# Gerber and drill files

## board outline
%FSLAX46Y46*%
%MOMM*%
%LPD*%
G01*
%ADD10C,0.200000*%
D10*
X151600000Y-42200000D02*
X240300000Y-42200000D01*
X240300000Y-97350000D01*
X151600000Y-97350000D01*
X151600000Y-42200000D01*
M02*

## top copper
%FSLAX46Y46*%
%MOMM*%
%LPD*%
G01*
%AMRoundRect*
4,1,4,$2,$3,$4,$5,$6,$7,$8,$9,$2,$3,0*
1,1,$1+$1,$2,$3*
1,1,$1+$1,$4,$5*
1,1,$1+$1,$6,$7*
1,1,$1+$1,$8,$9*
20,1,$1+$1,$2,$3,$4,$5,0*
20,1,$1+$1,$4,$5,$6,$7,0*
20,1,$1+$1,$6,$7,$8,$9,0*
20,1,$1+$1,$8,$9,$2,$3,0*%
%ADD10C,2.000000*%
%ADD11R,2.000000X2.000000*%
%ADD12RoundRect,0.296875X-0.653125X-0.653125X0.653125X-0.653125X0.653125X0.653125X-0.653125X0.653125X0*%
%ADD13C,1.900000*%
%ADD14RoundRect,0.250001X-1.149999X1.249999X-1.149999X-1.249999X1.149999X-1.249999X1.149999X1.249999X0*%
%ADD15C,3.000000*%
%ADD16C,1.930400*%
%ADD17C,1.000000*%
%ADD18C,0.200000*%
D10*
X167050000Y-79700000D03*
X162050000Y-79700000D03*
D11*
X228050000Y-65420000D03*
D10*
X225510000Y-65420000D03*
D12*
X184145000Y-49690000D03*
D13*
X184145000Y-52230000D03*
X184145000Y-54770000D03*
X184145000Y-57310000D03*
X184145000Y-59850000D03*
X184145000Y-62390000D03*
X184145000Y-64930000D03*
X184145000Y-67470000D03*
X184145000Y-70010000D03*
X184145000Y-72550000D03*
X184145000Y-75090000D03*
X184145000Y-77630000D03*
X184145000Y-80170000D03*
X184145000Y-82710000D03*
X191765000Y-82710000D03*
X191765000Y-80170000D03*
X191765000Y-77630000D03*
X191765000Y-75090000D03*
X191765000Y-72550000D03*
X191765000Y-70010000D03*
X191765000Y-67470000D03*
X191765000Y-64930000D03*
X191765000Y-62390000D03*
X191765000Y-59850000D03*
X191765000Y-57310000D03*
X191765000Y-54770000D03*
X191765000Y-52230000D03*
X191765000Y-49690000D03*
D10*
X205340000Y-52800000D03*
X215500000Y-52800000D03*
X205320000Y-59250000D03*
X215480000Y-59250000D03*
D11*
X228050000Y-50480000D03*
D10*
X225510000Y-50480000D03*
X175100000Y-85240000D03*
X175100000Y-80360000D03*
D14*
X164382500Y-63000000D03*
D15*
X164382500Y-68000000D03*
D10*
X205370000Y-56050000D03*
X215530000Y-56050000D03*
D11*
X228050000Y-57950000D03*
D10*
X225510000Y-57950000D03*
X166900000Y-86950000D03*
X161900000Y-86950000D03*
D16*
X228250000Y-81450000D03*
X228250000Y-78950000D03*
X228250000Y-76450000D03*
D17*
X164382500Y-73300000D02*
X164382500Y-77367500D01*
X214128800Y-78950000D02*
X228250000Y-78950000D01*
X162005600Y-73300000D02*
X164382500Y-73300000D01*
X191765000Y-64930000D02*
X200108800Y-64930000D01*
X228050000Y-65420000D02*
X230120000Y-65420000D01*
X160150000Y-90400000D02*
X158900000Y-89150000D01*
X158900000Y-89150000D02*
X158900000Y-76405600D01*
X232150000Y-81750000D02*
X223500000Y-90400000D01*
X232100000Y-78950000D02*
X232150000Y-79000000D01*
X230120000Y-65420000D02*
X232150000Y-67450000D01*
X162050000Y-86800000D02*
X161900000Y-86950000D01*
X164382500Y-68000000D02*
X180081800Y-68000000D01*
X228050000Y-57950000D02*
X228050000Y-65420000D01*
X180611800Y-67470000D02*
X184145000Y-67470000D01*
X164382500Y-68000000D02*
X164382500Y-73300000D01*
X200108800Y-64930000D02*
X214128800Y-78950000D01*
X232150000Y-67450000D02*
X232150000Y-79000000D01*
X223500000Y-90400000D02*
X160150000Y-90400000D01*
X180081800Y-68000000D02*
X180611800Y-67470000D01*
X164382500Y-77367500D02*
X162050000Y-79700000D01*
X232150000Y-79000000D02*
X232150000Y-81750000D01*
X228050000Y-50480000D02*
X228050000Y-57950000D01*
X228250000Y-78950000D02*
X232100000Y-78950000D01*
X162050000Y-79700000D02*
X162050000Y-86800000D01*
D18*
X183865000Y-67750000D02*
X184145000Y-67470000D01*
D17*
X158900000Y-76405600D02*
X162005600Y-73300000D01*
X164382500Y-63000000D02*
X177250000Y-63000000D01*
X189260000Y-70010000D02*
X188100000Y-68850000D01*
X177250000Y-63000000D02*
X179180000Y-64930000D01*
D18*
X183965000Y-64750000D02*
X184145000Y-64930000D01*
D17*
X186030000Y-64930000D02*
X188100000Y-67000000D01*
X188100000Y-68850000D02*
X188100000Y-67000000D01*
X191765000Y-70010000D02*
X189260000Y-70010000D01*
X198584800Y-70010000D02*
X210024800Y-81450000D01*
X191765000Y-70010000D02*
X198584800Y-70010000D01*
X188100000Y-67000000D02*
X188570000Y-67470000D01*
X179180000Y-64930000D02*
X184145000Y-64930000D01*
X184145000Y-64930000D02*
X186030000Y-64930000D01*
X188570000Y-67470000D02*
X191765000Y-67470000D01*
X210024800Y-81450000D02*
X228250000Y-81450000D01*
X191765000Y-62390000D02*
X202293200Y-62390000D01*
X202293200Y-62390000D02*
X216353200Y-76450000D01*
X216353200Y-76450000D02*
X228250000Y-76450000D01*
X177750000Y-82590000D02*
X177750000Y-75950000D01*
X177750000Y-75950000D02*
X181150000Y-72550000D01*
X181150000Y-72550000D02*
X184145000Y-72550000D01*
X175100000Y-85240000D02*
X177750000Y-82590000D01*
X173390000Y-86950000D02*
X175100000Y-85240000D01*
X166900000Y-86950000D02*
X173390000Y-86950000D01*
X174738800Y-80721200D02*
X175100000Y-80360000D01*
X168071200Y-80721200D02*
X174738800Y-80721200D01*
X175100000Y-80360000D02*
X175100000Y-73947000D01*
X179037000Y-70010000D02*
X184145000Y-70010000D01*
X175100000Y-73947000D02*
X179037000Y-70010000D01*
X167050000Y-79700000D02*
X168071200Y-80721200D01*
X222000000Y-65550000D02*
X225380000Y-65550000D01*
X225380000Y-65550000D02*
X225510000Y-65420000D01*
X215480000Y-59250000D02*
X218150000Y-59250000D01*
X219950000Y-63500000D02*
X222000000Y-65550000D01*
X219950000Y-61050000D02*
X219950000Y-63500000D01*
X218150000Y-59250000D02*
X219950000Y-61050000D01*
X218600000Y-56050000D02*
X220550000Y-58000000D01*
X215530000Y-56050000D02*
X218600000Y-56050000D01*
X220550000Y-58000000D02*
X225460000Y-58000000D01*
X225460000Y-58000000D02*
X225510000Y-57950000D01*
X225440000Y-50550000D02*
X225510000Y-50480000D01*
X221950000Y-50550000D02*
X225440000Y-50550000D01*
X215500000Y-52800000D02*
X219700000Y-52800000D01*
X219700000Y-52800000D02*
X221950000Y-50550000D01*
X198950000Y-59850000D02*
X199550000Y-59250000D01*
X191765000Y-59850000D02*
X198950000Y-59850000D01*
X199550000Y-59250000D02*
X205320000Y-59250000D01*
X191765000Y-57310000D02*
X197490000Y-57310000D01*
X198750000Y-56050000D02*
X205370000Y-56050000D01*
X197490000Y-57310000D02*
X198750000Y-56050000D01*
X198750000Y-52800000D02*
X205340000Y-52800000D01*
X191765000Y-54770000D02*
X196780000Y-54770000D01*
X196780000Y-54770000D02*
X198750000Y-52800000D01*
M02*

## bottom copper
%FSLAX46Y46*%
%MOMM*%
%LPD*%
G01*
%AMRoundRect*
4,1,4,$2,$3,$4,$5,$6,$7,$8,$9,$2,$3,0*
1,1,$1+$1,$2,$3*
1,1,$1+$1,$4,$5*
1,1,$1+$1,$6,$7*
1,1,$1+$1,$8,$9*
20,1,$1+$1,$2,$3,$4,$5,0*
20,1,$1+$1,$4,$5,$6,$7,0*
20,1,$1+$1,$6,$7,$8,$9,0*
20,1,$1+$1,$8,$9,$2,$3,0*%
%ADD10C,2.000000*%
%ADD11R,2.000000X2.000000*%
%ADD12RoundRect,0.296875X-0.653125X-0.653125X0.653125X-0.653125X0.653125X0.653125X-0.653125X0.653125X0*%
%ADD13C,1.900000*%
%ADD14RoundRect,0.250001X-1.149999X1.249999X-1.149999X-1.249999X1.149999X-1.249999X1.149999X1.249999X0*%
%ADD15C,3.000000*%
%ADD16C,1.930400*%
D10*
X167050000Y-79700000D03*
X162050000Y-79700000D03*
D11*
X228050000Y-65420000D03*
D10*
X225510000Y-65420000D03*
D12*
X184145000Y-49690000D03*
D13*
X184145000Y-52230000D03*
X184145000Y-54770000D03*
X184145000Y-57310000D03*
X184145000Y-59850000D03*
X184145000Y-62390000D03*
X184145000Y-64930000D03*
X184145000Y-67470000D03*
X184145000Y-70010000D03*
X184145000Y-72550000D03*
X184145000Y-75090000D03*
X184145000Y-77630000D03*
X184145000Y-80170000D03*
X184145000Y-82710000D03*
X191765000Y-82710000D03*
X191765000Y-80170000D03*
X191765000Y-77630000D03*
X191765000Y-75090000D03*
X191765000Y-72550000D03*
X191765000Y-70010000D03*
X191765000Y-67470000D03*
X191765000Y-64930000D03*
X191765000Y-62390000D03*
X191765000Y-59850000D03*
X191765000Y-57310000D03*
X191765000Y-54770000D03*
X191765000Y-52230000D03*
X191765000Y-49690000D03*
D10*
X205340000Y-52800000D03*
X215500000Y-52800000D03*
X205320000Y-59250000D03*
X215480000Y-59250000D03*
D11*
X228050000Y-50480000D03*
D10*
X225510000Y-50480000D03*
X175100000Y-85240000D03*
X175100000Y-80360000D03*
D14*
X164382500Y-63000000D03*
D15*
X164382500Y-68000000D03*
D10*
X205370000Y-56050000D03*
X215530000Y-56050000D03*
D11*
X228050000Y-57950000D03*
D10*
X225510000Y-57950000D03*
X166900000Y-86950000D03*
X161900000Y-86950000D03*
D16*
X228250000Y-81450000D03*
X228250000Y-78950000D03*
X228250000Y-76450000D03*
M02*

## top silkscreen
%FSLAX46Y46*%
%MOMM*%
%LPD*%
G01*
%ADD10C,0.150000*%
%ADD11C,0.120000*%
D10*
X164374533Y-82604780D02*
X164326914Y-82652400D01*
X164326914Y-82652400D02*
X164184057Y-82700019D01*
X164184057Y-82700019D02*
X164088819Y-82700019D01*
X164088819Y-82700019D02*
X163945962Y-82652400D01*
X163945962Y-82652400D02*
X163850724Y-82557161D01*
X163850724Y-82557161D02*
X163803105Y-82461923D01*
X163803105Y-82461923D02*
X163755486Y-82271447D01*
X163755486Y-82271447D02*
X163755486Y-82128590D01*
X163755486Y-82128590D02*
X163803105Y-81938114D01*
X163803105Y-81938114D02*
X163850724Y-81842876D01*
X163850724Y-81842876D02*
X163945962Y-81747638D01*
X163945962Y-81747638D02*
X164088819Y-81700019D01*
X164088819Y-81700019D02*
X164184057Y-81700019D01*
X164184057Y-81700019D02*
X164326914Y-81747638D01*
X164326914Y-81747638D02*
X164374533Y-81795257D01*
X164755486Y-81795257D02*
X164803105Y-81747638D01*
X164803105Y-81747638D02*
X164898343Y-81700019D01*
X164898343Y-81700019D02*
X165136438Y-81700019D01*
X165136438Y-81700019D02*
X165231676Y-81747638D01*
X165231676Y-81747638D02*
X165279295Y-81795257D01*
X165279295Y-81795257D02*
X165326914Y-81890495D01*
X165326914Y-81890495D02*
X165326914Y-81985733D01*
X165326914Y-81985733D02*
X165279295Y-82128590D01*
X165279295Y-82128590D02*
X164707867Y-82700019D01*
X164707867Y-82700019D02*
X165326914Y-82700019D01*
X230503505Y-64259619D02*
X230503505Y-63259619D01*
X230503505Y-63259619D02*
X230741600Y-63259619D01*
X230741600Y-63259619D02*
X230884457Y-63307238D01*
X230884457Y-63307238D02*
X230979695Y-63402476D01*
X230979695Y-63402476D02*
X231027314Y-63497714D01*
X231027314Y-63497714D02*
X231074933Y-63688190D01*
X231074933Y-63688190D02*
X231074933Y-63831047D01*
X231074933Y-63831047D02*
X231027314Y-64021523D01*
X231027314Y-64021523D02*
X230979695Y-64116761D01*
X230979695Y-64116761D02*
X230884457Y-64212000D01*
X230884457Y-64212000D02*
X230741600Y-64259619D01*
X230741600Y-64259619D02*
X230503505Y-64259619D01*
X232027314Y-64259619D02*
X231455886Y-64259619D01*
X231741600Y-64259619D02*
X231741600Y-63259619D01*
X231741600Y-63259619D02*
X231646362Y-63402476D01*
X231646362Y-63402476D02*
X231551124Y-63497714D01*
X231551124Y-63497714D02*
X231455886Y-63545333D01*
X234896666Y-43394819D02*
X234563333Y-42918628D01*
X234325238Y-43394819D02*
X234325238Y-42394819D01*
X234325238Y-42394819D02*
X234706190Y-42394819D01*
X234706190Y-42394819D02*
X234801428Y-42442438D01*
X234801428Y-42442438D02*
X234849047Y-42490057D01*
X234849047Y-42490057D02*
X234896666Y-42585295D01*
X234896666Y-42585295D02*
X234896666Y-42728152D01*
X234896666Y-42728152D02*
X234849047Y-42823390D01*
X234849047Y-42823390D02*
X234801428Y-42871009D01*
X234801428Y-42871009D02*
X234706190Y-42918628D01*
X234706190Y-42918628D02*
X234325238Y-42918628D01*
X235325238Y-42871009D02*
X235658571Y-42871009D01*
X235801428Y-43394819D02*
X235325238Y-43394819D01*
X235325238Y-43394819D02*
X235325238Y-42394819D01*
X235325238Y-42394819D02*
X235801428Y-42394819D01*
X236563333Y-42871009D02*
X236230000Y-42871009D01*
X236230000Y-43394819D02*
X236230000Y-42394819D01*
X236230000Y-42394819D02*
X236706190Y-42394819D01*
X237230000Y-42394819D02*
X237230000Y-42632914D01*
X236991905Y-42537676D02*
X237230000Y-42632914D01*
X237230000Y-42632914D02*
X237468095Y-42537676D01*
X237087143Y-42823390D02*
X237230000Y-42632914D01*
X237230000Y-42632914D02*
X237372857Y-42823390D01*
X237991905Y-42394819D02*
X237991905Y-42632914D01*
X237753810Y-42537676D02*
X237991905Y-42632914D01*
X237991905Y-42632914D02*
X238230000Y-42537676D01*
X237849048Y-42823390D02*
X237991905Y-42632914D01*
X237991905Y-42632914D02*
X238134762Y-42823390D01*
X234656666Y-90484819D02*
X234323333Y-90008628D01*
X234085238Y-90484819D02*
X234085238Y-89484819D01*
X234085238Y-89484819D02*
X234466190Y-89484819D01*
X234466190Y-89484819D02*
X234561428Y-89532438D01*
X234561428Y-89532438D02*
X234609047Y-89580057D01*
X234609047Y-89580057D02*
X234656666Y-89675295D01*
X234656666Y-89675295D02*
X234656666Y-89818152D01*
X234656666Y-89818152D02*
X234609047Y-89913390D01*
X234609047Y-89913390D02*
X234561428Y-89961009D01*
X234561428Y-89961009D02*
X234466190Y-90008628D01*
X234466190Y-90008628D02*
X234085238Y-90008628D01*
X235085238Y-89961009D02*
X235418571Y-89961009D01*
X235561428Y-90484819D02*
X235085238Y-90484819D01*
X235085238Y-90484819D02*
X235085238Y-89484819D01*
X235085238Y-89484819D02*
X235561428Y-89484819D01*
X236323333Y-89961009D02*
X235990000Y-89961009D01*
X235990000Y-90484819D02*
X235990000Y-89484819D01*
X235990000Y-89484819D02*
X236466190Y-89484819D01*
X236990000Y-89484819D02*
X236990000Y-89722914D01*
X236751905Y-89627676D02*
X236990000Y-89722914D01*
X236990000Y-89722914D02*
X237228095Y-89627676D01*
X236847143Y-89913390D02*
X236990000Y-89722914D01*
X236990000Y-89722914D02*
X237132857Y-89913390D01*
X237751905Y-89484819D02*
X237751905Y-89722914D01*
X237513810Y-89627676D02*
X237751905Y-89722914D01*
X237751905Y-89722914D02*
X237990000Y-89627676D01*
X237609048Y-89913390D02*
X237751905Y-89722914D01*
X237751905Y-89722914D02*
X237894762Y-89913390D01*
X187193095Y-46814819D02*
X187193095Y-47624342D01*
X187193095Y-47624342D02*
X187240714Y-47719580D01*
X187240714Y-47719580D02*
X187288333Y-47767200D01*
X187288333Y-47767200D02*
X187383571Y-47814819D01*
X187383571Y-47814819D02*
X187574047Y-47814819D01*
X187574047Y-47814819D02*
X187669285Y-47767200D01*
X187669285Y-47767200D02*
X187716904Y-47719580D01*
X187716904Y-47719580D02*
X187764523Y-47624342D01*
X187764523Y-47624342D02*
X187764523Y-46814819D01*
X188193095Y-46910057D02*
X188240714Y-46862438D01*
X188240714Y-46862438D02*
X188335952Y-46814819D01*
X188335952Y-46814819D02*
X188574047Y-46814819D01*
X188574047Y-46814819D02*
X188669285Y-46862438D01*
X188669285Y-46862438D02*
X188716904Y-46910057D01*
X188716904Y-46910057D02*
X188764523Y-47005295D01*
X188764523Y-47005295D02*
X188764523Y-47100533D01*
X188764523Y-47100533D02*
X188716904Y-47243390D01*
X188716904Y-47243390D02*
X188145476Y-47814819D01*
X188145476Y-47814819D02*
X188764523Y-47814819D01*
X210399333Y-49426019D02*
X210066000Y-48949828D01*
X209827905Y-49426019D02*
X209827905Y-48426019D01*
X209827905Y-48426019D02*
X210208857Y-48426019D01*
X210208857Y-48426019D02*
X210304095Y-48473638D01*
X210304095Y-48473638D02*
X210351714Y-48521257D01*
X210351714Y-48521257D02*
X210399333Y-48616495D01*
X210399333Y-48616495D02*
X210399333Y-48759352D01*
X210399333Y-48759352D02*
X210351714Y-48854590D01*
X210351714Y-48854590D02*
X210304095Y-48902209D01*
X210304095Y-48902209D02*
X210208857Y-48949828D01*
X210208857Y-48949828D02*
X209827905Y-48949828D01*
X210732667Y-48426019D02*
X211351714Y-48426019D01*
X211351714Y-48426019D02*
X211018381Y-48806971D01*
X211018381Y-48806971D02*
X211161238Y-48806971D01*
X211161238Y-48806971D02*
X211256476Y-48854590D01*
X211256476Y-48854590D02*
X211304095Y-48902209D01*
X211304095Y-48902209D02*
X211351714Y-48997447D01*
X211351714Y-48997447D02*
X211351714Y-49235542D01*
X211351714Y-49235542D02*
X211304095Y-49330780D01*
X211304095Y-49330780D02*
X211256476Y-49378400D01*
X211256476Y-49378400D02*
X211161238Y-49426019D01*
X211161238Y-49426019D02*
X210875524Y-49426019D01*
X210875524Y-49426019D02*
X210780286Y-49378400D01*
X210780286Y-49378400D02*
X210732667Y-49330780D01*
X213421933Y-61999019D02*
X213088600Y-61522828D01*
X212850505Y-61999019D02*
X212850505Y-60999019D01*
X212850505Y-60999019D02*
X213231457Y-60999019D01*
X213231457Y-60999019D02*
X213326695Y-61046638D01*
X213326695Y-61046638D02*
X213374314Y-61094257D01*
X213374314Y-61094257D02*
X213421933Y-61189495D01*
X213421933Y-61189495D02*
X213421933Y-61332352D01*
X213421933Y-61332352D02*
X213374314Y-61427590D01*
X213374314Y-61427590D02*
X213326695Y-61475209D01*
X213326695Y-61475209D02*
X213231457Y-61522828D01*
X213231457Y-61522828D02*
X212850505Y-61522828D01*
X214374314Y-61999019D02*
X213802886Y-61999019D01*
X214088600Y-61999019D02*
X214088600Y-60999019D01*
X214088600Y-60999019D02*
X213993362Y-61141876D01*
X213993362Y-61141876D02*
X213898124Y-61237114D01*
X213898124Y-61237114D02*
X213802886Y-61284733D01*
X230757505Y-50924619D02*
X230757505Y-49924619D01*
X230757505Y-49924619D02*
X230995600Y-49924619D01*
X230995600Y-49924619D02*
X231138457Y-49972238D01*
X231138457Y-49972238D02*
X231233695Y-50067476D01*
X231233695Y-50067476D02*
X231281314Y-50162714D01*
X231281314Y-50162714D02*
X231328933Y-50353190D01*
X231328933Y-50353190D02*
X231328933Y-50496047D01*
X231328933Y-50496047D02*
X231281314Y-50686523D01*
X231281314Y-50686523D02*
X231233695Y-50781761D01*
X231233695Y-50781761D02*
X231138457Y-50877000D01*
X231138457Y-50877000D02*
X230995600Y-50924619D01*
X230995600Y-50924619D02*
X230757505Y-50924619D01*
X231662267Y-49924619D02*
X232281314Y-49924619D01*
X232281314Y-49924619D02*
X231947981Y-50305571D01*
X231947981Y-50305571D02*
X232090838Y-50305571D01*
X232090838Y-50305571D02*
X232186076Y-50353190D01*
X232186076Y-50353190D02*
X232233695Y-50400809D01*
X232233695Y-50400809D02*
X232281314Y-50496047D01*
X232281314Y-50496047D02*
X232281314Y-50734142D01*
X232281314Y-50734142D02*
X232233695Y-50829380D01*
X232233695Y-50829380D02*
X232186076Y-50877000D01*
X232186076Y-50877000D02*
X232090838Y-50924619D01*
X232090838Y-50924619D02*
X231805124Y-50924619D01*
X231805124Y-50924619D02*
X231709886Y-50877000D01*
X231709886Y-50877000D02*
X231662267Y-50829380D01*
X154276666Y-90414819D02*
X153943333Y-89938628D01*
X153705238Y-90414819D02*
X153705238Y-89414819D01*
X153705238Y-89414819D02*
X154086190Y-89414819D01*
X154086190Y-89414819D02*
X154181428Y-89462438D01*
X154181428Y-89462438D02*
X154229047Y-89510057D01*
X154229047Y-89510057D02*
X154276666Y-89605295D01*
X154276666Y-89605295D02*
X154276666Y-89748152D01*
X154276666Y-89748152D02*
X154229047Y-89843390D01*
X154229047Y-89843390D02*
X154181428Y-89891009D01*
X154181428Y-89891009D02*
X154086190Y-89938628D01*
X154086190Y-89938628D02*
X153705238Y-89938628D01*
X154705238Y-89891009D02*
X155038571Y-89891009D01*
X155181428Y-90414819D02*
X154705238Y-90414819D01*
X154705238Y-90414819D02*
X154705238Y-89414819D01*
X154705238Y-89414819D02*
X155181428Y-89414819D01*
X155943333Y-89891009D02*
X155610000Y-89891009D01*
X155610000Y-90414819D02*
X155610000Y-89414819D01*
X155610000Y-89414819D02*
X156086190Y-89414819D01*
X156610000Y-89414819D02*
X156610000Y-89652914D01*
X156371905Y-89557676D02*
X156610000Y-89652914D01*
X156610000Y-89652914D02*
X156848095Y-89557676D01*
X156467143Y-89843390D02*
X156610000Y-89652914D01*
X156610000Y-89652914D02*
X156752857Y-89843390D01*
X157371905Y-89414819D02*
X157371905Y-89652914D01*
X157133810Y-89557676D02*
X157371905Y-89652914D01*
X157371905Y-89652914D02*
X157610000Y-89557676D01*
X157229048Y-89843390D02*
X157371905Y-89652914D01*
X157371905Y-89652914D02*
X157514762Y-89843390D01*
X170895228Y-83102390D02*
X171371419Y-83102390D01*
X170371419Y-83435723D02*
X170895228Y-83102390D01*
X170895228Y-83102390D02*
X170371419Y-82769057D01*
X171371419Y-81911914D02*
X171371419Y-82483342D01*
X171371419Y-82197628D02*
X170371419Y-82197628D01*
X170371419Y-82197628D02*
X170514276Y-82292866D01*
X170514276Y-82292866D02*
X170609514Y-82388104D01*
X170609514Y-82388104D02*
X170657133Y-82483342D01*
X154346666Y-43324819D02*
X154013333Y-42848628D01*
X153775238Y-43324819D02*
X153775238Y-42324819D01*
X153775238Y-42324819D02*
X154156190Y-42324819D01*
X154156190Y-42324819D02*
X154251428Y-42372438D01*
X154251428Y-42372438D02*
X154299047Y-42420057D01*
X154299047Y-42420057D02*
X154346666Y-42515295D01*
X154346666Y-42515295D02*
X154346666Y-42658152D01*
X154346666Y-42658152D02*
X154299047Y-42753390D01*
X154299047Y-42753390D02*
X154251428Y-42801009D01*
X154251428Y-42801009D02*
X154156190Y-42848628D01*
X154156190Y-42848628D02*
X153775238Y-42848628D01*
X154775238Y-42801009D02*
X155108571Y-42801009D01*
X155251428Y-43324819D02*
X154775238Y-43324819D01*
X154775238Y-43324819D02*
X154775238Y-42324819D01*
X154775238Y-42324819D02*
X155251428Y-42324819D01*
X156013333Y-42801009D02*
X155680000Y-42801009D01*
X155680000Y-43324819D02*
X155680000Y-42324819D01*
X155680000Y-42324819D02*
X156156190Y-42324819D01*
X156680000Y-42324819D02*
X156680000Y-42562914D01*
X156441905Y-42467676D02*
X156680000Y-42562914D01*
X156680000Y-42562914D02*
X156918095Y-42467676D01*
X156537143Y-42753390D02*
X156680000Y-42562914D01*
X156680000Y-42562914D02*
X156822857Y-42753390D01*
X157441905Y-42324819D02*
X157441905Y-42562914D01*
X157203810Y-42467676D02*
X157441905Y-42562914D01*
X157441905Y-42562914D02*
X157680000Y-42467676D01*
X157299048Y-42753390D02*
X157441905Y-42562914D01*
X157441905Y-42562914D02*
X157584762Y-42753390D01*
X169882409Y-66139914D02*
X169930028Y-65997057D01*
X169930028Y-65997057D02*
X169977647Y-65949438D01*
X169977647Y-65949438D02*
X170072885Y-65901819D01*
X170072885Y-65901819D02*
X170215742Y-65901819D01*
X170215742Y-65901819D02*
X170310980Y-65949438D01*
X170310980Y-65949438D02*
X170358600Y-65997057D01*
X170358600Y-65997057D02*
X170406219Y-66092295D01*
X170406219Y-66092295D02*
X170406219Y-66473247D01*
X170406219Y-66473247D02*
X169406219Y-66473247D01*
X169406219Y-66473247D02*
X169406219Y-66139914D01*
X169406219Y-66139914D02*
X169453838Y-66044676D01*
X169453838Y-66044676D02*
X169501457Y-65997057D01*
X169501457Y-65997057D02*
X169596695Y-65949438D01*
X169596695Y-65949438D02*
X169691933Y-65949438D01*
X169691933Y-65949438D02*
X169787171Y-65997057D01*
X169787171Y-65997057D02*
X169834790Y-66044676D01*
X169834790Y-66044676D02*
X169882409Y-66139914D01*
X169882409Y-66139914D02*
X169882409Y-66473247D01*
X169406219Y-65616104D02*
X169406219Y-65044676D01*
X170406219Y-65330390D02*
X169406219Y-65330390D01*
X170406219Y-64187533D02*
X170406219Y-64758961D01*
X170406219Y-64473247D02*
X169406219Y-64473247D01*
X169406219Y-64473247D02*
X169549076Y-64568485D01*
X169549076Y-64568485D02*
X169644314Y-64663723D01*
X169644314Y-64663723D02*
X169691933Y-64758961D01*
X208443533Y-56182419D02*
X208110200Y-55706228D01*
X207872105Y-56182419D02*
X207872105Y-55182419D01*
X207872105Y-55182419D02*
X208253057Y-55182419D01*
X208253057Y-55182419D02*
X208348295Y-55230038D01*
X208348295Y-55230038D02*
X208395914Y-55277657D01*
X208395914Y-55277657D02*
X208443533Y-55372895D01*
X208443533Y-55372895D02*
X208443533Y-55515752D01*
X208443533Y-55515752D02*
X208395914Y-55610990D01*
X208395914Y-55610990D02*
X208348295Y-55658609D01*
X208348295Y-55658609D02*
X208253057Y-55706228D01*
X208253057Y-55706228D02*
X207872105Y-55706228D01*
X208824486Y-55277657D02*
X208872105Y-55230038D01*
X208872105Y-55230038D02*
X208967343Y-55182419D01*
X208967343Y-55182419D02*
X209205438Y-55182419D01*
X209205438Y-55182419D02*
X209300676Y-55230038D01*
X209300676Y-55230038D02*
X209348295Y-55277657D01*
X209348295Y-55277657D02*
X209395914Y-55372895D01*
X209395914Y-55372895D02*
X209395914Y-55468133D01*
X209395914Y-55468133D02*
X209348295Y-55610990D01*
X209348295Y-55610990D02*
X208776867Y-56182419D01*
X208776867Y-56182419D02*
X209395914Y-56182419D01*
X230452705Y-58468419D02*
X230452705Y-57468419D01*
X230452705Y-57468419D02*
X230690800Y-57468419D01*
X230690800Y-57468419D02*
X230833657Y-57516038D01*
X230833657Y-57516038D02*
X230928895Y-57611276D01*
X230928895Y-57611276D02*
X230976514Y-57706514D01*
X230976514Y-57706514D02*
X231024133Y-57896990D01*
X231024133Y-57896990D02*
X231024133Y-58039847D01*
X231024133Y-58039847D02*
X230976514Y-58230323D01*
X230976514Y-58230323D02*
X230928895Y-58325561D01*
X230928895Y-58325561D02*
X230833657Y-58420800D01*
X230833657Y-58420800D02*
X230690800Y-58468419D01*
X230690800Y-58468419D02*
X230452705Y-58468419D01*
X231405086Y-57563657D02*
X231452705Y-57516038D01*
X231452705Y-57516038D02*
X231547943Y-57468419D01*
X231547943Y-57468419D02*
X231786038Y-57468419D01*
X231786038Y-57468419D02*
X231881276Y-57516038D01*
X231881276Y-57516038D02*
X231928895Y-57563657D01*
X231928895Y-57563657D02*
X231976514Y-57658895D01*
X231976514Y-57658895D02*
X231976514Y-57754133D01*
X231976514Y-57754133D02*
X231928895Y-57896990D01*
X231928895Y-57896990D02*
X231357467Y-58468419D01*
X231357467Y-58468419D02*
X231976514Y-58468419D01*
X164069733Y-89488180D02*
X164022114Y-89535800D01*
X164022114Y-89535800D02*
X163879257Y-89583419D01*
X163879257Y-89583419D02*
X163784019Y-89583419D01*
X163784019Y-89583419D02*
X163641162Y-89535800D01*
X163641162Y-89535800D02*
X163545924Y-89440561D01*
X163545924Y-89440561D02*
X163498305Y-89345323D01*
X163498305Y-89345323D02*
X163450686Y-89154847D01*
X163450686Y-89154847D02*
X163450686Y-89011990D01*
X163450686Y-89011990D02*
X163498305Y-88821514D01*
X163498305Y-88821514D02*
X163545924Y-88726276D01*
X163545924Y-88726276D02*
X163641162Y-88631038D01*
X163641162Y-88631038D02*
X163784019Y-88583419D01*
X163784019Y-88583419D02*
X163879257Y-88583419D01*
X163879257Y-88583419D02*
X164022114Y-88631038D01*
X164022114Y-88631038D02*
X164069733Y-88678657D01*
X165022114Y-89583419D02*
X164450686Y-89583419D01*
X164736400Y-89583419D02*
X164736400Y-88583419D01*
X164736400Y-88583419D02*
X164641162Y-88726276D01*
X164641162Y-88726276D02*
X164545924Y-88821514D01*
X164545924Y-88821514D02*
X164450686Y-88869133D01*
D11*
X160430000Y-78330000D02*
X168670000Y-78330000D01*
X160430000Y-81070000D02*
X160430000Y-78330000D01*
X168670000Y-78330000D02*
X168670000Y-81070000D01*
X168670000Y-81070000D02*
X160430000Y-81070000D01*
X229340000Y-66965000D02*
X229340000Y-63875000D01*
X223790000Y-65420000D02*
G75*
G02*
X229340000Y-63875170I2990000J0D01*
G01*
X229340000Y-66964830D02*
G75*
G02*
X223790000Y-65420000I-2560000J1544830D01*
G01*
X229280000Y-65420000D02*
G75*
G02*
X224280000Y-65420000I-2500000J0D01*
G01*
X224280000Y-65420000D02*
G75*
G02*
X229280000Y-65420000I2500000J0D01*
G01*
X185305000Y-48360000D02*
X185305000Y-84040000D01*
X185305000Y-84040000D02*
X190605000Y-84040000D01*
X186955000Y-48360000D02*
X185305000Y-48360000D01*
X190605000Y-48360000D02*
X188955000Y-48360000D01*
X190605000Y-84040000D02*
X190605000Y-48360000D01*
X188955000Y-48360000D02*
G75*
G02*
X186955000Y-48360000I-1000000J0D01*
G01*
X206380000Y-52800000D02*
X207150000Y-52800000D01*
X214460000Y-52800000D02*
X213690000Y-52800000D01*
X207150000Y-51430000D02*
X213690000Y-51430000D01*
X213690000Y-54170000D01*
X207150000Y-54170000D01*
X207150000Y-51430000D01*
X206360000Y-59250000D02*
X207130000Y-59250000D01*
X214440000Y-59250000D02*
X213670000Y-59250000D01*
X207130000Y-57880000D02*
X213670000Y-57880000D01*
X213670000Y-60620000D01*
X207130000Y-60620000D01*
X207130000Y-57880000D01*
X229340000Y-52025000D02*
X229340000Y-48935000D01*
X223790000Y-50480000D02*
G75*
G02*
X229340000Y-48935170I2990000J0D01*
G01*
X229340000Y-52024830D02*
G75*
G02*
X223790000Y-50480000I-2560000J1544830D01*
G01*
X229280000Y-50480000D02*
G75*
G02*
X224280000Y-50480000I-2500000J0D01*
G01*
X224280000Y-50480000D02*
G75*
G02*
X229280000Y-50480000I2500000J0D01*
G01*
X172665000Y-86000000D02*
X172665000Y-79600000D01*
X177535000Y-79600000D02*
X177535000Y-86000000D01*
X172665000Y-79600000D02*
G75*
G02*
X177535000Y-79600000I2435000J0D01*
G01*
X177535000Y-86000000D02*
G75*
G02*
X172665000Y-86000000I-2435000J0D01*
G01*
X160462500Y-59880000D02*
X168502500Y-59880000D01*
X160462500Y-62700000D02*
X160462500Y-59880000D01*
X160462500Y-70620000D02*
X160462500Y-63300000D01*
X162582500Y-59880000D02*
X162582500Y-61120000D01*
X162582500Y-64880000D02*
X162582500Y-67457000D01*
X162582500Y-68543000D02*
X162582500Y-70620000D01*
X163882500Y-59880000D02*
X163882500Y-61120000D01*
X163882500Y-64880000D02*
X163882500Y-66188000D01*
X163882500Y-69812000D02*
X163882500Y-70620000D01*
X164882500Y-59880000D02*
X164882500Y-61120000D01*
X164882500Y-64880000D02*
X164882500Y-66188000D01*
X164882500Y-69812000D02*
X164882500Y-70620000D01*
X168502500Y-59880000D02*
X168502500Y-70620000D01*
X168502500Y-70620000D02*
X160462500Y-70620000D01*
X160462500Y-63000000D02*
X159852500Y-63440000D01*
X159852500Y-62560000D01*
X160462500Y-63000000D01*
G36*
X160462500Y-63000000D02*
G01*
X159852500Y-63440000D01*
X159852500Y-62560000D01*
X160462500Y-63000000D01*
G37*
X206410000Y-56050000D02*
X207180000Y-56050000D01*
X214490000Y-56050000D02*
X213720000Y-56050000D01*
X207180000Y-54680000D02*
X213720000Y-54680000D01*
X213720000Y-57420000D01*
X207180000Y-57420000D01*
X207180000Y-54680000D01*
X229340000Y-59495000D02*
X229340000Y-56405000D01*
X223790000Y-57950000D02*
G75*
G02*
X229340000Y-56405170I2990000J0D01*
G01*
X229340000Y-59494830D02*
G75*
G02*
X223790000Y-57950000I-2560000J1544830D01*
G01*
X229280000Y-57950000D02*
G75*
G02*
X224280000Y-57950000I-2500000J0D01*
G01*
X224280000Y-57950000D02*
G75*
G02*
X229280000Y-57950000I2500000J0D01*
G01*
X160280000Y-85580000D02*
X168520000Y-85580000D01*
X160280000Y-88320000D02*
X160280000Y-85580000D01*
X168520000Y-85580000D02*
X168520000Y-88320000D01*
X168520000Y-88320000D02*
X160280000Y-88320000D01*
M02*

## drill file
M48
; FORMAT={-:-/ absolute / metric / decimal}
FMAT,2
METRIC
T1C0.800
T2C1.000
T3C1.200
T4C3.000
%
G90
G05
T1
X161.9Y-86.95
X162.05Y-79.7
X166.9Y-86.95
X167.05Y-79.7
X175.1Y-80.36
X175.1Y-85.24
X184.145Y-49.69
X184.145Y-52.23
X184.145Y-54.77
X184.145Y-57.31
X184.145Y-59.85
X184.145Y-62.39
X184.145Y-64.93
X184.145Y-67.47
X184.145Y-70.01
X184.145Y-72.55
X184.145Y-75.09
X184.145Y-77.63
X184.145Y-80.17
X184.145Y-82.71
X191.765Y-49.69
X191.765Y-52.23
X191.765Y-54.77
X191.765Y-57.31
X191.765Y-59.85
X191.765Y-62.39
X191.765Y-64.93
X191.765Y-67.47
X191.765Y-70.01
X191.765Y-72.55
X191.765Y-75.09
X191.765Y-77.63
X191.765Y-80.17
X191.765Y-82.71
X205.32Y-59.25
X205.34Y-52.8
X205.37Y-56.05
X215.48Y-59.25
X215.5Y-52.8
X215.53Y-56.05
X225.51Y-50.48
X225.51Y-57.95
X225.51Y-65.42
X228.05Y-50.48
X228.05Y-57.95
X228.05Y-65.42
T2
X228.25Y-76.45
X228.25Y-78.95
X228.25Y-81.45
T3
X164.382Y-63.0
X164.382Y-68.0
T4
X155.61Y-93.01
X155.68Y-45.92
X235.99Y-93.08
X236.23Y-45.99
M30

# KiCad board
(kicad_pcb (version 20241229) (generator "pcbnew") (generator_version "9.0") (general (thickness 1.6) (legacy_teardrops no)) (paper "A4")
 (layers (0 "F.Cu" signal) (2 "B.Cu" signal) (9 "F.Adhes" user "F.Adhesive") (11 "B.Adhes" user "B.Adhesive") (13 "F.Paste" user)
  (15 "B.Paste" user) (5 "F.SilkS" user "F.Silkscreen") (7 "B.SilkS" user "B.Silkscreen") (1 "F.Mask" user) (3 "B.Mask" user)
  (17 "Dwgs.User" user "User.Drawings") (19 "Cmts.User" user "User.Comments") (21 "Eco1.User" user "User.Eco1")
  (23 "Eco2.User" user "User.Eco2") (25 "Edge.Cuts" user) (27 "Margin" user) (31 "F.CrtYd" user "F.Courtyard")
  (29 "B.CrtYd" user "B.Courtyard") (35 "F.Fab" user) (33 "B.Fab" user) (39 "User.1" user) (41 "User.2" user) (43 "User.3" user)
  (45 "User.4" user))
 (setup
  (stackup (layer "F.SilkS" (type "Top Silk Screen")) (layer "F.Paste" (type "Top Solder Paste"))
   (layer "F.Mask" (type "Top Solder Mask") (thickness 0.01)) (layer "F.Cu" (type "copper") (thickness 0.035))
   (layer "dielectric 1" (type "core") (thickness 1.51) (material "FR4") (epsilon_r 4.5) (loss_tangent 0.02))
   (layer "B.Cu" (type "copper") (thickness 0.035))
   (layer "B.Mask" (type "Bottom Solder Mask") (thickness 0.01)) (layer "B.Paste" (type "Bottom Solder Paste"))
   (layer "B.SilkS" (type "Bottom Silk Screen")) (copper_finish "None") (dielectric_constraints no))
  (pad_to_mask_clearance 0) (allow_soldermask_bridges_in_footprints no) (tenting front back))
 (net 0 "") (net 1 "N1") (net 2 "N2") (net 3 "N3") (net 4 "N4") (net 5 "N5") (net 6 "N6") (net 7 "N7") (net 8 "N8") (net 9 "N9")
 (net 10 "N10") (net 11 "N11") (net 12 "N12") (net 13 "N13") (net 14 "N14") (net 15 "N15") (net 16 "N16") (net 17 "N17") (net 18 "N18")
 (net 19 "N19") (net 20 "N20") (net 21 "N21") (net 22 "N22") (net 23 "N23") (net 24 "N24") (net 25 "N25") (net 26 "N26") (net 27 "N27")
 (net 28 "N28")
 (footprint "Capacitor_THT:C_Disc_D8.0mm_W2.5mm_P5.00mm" (layer "F.Cu") (at 167.05 79.7 180)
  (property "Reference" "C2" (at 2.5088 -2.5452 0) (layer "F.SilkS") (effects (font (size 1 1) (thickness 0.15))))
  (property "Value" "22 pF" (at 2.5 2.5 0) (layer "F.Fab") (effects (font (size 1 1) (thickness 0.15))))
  (fp_line (start 6.62 1.37) (end -1.62 1.37) (stroke (width 0.12) (type solid)) (layer "F.SilkS"))
  (fp_line (start 6.62 -1.37) (end 6.62 1.37) (stroke (width 0.12) (type solid)) (layer "F.SilkS"))
  (fp_line (start -1.62 1.37) (end -1.62 -1.37) (stroke (width 0.12) (type solid)) (layer "F.SilkS"))
  (fp_line (start -1.62 -1.37) (end 6.62 -1.37) (stroke (width 0.12) (type solid)) (layer "F.SilkS"))
  (pad "1" thru_hole circle (at 0 0 180) (size 2 2) (drill 0.8) (layers "*.Cu" "*.Mask") (remove_unused_layers no) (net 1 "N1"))
  (pad "2" thru_hole circle (at 5 0 180) (size 2 2) (drill 0.8) (layers "*.Cu" "*.Mask") (remove_unused_layers no) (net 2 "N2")))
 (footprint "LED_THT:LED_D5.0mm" (layer "F.Cu") (at 228.05 65.42 180)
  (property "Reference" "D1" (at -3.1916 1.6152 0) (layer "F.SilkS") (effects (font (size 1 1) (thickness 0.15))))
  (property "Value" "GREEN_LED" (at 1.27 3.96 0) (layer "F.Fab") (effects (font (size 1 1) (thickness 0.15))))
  (fp_line (start -1.29 -1.545) (end -1.29 1.545) (stroke (width 0.12) (type solid)) (layer "F.SilkS"))
  (fp_arc (start 4.26 0) (mid 2.071779 2.880495) (end -1.29 1.54483) (stroke (width 0.12) (type solid)) (layer "F.SilkS"))
  (fp_arc (start -1.29 -1.54483) (mid 2.071779 -2.880495) (end 4.26 0) (stroke (width 0.12) (type solid)) (layer "F.SilkS"))
  (fp_circle (center 1.27 0) (end 3.77 0) (stroke (width 0.12) (type solid)) (fill no) (layer "F.SilkS"))
  (pad "1" thru_hole rect (at 0 0 180) (size 2 2) (drill 0.8) (layers "*.Cu" "*.Mask") (remove_unused_layers no) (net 2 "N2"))
  (pad "2" thru_hole circle (at 2.54 0 180) (size 2 2) (drill 0.8) (layers "*.Cu" "*.Mask") (remove_unused_layers no) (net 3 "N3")))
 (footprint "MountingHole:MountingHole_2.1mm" (layer "F.Cu") (at 236.23 45.99)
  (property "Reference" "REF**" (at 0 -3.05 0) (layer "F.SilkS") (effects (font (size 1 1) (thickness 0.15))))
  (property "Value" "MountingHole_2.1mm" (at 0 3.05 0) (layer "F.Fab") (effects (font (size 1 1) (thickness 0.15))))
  (pad "" np_thru_hole circle (at 0 0) (size 2.1 2.1) (drill 3) (layers "*.Cu" "*.Mask")))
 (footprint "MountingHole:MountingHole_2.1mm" (layer "F.Cu") (at 235.99 93.08)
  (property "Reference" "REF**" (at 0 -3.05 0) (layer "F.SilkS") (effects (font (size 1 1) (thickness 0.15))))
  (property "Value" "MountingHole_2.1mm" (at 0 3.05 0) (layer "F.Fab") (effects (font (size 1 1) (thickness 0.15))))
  (pad "" np_thru_hole circle (at 0 0) (size 2.1 2.1) (drill 3) (layers "*.Cu" "*.Mask")))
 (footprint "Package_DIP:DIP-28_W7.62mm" (layer "F.Cu") (at 184.145 49.69)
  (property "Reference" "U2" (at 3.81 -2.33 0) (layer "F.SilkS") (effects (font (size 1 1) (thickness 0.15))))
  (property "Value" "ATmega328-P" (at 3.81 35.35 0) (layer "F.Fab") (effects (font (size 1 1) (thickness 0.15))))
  (fp_line (start 1.16 -1.33) (end 1.16 34.35) (stroke (width 0.12) (type solid)) (layer "F.SilkS"))
  (fp_line (start 1.16 34.35) (end 6.46 34.35) (stroke (width 0.12) (type solid)) (layer "F.SilkS"))
  (fp_line (start 2.81 -1.33) (end 1.16 -1.33) (stroke (width 0.12) (type solid)) (layer "F.SilkS"))
  (fp_line (start 6.46 -1.33) (end 4.81 -1.33) (stroke (width 0.12) (type solid)) (layer "F.SilkS"))
  (fp_line (start 6.46 34.35) (end 6.46 -1.33) (stroke (width 0.12) (type solid)) (layer "F.SilkS"))
  (fp_arc (start 4.81 -1.33) (mid 3.81 -0.33) (end 2.81 -1.33) (stroke (width 0.12) (type solid)) (layer "F.SilkS"))
  (pad "1" thru_hole roundrect (at 0 0) (size 1.9 1.9) (drill 0.8) (layers "*.Cu" "*.Mask") (remove_unused_layers no)
   (roundrect_rratio 0.15625) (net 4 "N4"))
  (pad "2" thru_hole circle (at 0 2.54) (size 1.9 1.9) (drill 0.8) (layers "*.Cu" "*.Mask") (remove_unused_layers no) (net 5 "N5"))
  (pad "3" thru_hole circle (at 0 5.08) (size 1.9 1.9) (drill 0.8) (layers "*.Cu" "*.Mask") (remove_unused_layers no) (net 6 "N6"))
  (pad "4" thru_hole circle (at 0 7.62) (size 1.9 1.9) (drill 0.8) (layers "*.Cu" "*.Mask") (remove_unused_layers no) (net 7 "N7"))
  (pad "5" thru_hole circle (at 0 10.16) (size 1.9 1.9) (drill 0.8) (layers "*.Cu" "*.Mask") (remove_unused_layers no) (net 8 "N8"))
  (pad "6" thru_hole circle (at 0 12.7) (size 1.9 1.9) (drill 0.8) (layers "*.Cu" "*.Mask") (remove_unused_layers no) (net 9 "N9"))
  (pad "7" thru_hole circle (at 0 15.24) (size 1.9 1.9) (drill 0.8) (layers "*.Cu" "*.Mask") (remove_unused_layers no) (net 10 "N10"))
  (pad "8" thru_hole circle (at 0 17.78) (size 1.9 1.9) (drill 0.8) (layers "*.Cu" "*.Mask") (remove_unused_layers no) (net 2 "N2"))
  (pad "9" thru_hole circle (at 0 20.32) (size 1.9 1.9) (drill 0.8) (layers "*.Cu" "*.Mask") (remove_unused_layers no) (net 1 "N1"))
  (pad "10" thru_hole circle (at 0 22.86) (size 1.9 1.9) (drill 0.8) (layers "*.Cu" "*.Mask") (remove_unused_layers no) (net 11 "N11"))
  (pad "11" thru_hole circle (at 0 25.4) (size 1.9 1.9) (drill 0.8) (layers "*.Cu" "*.Mask") (remove_unused_layers no) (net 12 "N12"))
  (pad "12" thru_hole circle (at 0 27.94) (size 1.9 1.9) (drill 0.8) (layers "*.Cu" "*.Mask") (remove_unused_layers no) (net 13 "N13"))
  (pad "13" thru_hole circle (at 0 30.48) (size 1.9 1.9) (drill 0.8) (layers "*.Cu" "*.Mask") (remove_unused_layers no) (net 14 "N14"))
  (pad "14" thru_hole circle (at 0 33.02) (size 1.9 1.9) (drill 0.8) (layers "*.Cu" "*.Mask") (remove_unused_layers no) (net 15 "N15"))
  (pad "15" thru_hole circle (at 7.62 33.02) (size 1.9 1.9) (drill 0.8) (layers "*.Cu" "*.Mask") (remove_unused_layers no) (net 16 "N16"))
  (pad "16" thru_hole circle (at 7.62 30.48) (size 1.9 1.9) (drill 0.8) (layers "*.Cu" "*.Mask") (remove_unused_layers no) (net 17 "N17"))
  (pad "17" thru_hole circle (at 7.62 27.94) (size 1.9 1.9) (drill 0.8) (layers "*.Cu" "*.Mask") (remove_unused_layers no) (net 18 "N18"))
  (pad "18" thru_hole circle (at 7.62 25.4) (size 1.9 1.9) (drill 0.8) (layers "*.Cu" "*.Mask") (remove_unused_layers no) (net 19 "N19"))
  (pad "19" thru_hole circle (at 7.62 22.86) (size 1.9 1.9) (drill 0.8) (layers "*.Cu" "*.Mask") (remove_unused_layers no) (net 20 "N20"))
  (pad "20" thru_hole circle (at 7.62 20.32) (size 1.9 1.9) (drill 0.8) (layers "*.Cu" "*.Mask") (remove_unused_layers no) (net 10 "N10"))
  (pad "21" thru_hole circle (at 7.62 17.78) (size 1.9 1.9) (drill 0.8) (layers "*.Cu" "*.Mask") (remove_unused_layers no) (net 10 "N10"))
  (pad "22" thru_hole circle (at 7.62 15.24) (size 1.9 1.9) (drill 0.8) (layers "*.Cu" "*.Mask") (remove_unused_layers no) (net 2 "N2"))
  (pad "23" thru_hole circle (at 7.62 12.7) (size 1.9 1.9) (drill 0.8) (layers "*.Cu" "*.Mask") (remove_unused_layers no) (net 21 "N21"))
  (pad "24" thru_hole circle (at 7.62 10.16) (size 1.9 1.9) (drill 0.8) (layers "*.Cu" "*.Mask") (remove_unused_layers no) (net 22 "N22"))
  (pad "25" thru_hole circle (at 7.62 7.62) (size 1.9 1.9) (drill 0.8) (layers "*.Cu" "*.Mask") (remove_unused_layers no) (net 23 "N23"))
  (pad "26" thru_hole circle (at 7.62 5.08) (size 1.9 1.9) (drill 0.8) (layers "*.Cu" "*.Mask") (remove_unused_layers no) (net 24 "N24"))
  (pad "27" thru_hole circle (at 7.62 2.54) (size 1.9 1.9) (drill 0.8) (layers "*.Cu" "*.Mask") (remove_unused_layers no) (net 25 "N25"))
  (pad "28" thru_hole circle (at 7.62 0) (size 1.9 1.9) (drill 0.8) (layers "*.Cu" "*.Mask") (remove_unused_layers no) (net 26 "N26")))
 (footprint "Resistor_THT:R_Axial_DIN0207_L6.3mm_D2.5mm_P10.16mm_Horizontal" (layer "F.Cu") (at 205.34 52.8)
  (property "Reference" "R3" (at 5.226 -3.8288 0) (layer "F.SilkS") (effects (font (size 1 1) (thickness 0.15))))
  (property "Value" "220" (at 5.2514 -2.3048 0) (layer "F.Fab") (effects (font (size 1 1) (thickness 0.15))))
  (fp_line (start 1.04 0) (end 1.81 0) (stroke (width 0.12) (type solid)) (layer "F.SilkS"))
  (fp_line (start 9.12 0) (end 8.35 0) (stroke (width 0.12) (type solid)) (layer "F.SilkS"))
  (fp_rect (start 1.81 -1.37) (end 8.35 1.37) (stroke (width 0.12) (type solid)) (fill no) (layer "F.SilkS"))
  (pad "1" thru_hole circle (at 0 0) (size 2 2) (drill 0.8) (layers "*.Cu" "*.Mask") (remove_unused_layers no) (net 24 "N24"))
  (pad "2" thru_hole circle (at 10.16 0) (size 2 2) (drill 0.8) (layers "*.Cu" "*.Mask") (remove_unused_layers no) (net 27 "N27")))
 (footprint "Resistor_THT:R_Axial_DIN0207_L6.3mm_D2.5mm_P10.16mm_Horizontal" (layer "F.Cu") (at 205.32 59.25)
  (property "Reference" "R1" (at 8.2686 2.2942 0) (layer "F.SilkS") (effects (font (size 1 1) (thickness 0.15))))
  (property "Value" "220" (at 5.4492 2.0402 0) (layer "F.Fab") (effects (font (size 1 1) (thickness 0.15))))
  (fp_line (start 1.04 0) (end 1.81 0) (stroke (width 0.12) (type solid)) (layer "F.SilkS"))
  (fp_line (start 9.12 0) (end 8.35 0) (stroke (width 0.12) (type solid)) (layer "F.SilkS"))
  (fp_rect (start 1.81 -1.37) (end 8.35 1.37) (stroke (width 0.12) (type solid)) (fill no) (layer "F.SilkS"))
  (pad "1" thru_hole circle (at 0 0) (size 2 2) (drill 0.8) (layers "*.Cu" "*.Mask") (remove_unused_layers no) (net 22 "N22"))
  (pad "2" thru_hole circle (at 10.16 0) (size 2 2) (drill 0.8) (layers "*.Cu" "*.Mask") (remove_unused_layers no) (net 3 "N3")))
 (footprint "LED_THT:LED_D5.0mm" (layer "F.Cu") (at 228.05 50.48 180)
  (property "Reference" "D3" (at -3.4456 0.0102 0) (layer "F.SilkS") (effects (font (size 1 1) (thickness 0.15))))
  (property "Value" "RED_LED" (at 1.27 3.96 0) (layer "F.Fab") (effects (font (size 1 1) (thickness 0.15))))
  (fp_line (start -1.29 -1.545) (end -1.29 1.545) (stroke (width 0.12) (type solid)) (layer "F.SilkS"))
  (fp_arc (start 4.26 0) (mid 2.071779 2.880495) (end -1.29 1.54483) (stroke (width 0.12) (type solid)) (layer "F.SilkS"))
  (fp_arc (start -1.29 -1.54483) (mid 2.071779 -2.880495) (end 4.26 0) (stroke (width 0.12) (type solid)) (layer "F.SilkS"))
  (fp_circle (center 1.27 0) (end 3.77 0) (stroke (width 0.12) (type solid)) (fill no) (layer "F.SilkS"))
  (pad "1" thru_hole rect (at 0 0 180) (size 2 2) (drill 0.8) (layers "*.Cu" "*.Mask") (remove_unused_layers no) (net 2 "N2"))
  (pad "2" thru_hole circle (at 2.54 0 180) (size 2 2) (drill 0.8) (layers "*.Cu" "*.Mask") (remove_unused_layers no) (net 27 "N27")))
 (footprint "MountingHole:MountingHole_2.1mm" (layer "F.Cu") (at 155.61 93.01)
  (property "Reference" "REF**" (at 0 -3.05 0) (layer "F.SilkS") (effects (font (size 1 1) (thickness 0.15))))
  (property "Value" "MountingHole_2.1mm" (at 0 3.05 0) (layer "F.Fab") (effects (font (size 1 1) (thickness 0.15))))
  (pad "" np_thru_hole circle (at 0 0) (size 2.1 2.1) (drill 3) (layers "*.Cu" "*.Mask")))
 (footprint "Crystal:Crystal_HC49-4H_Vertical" (layer "F.Cu") (at 175.1 85.24 90)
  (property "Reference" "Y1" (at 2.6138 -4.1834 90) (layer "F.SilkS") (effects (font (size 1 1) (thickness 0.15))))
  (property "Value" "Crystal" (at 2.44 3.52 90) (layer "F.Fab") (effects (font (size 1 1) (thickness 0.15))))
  (fp_line (start -0.76 -2.435) (end 5.64 -2.435) (stroke (width 0.12) (type solid)) (layer "F.SilkS"))
  (fp_line (start 5.64 2.435) (end -0.76 2.435) (stroke (width 0.12) (type solid)) (layer "F.SilkS"))
  (fp_arc (start 5.64 -2.435) (mid 8.075 0) (end 5.64 2.435) (stroke (width 0.12) (type solid)) (layer "F.SilkS"))
  (fp_arc (start -0.76 2.435) (mid -3.195 0) (end -0.76 -2.435) (stroke (width 0.12) (type solid)) (layer "F.SilkS"))
  (pad "1" thru_hole circle (at 0 0 90) (size 2 2) (drill 0.8) (layers "*.Cu" "*.Mask") (remove_unused_layers no) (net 11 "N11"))
  (pad "2" thru_hole circle (at 4.88 0 90) (size 2 2) (drill 0.8) (layers "*.Cu" "*.Mask") (remove_unused_layers no) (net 1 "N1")))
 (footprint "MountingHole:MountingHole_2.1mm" (layer "F.Cu") (at 155.68 45.92)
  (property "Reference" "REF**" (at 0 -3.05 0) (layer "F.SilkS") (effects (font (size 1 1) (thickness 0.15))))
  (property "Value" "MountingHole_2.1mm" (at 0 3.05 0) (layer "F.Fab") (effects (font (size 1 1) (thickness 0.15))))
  (pad "" np_thru_hole circle (at 0 0) (size 2.1 2.1) (drill 3) (layers "*.Cu" "*.Mask")))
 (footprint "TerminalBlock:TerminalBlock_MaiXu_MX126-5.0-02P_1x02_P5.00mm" (layer "F.Cu") (at 164.3825 63 -90)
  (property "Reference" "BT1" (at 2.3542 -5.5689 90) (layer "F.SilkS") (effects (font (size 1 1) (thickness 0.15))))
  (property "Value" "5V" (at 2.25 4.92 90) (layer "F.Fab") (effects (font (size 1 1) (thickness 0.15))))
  (fp_line (start -3.12 3.92) (end -3.12 -4.12) (stroke (width 0.12) (type solid)) (layer "F.SilkS"))
  (fp_line (start -0.3 3.92) (end -3.12 3.92) (stroke (width 0.12) (type solid)) (layer "F.SilkS"))
  (fp_line (start 7.62 3.92) (end 0.3 3.92) (stroke (width 0.12) (type solid)) (layer "F.SilkS"))
  (fp_line (start -3.12 1.8) (end -1.88 1.8) (stroke (width 0.12) (type solid)) (layer "F.SilkS"))
  (fp_line (start 1.88 1.8) (end 4.457 1.8) (stroke (width 0.12) (type solid)) (layer "F.SilkS"))
  (fp_line (start 5.543 1.8) (end 7.62 1.8) (stroke (width 0.12) (type solid)) (layer "F.SilkS"))
  (fp_line (start -3.12 0.5) (end -1.88 0.5) (stroke (width 0.12) (type solid)) (layer "F.SilkS"))
  (fp_line (start 1.88 0.5) (end 3.188 0.5) (stroke (width 0.12) (type solid)) (layer "F.SilkS"))
  (fp_line (start 6.812 0.5) (end 7.62 0.5) (stroke (width 0.12) (type solid)) (layer "F.SilkS"))
  (fp_line (start -3.12 -0.5) (end -1.88 -0.5) (stroke (width 0.12) (type solid)) (layer "F.SilkS"))
  (fp_line (start 1.88 -0.5) (end 3.188 -0.5) (stroke (width 0.12) (type solid)) (layer "F.SilkS"))
  (fp_line (start 6.812 -0.5) (end 7.62 -0.5) (stroke (width 0.12) (type solid)) (layer "F.SilkS"))
  (fp_line (start -3.12 -4.12) (end 7.62 -4.12) (stroke (width 0.12) (type solid)) (layer "F.SilkS"))
  (fp_line (start 7.62 -4.12) (end 7.62 3.92) (stroke (width 0.12) (type solid)) (layer "F.SilkS"))
  (fp_poly (pts (xy 0 3.92) (xy 0.44 4.53) (xy -0.44 4.53)) (stroke (width 0.12) (type solid)) (fill yes) (layer "F.SilkS"))
  (pad "1" thru_hole roundrect (at 0 0 270) (size 3 2.8) (drill 1.2) (layers "*.Cu" "*.Mask") (remove_unused_layers no)
   (roundrect_rratio 0.089286) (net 10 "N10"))
  (pad "2" thru_hole circle (at 5 0 270) (size 3 3) (drill 1.2) (layers "*.Cu" "*.Mask") (remove_unused_layers no) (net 2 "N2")))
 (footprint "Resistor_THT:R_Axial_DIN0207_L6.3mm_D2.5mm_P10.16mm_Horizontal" (layer "F.Cu") (at 205.37 56.05)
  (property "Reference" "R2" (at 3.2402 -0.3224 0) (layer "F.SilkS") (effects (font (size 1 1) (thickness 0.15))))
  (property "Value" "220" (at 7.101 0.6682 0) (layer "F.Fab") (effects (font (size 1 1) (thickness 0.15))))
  (fp_line (start 1.04 0) (end 1.81 0) (stroke (width 0.12) (type solid)) (layer "F.SilkS"))
  (fp_line (start 9.12 0) (end 8.35 0) (stroke (width 0.12) (type solid)) (layer "F.SilkS"))
  (fp_rect (start 1.81 -1.37) (end 8.35 1.37) (stroke (width 0.12) (type solid)) (fill no) (layer "F.SilkS"))
  (pad "1" thru_hole circle (at 0 0) (size 2 2) (drill 0.8) (layers "*.Cu" "*.Mask") (remove_unused_layers no) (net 23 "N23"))
  (pad "2" thru_hole circle (at 10.16 0) (size 2 2) (drill 0.8) (layers "*.Cu" "*.Mask") (remove_unused_layers no) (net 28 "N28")))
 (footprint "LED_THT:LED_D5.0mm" (layer "F.Cu") (at 228.05 57.95 180)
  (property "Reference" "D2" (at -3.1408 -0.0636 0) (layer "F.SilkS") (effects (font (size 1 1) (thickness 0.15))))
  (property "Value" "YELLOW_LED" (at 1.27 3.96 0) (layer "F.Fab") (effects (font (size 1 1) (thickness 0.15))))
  (fp_line (start -1.29 -1.545) (end -1.29 1.545) (stroke (width 0.12) (type solid)) (layer "F.SilkS"))
  (fp_arc (start 4.26 0) (mid 2.071779 2.880495) (end -1.29 1.54483) (stroke (width 0.12) (type solid)) (layer "F.SilkS"))
  (fp_arc (start -1.29 -1.54483) (mid 2.071779 -2.880495) (end 4.26 0) (stroke (width 0.12) (type solid)) (layer "F.SilkS"))
  (fp_circle (center 1.27 0) (end 3.77 0) (stroke (width 0.12) (type solid)) (fill no) (layer "F.SilkS"))
  (pad "1" thru_hole rect (at 0 0 180) (size 2 2) (drill 0.8) (layers "*.Cu" "*.Mask") (remove_unused_layers no) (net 2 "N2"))
  (pad "2" thru_hole circle (at 2.54 0 180) (size 2 2) (drill 0.8) (layers "*.Cu" "*.Mask") (remove_unused_layers no) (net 28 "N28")))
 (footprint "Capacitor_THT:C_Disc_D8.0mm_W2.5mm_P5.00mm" (layer "F.Cu") (at 166.9 86.95 180)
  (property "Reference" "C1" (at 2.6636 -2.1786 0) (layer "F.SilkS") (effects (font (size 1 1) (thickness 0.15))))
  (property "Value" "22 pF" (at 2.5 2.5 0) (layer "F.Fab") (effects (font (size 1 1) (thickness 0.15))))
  (fp_line (start 6.62 1.37) (end -1.62 1.37) (stroke (width 0.12) (type solid)) (layer "F.SilkS"))
  (fp_line (start 6.62 -1.37) (end 6.62 1.37) (stroke (width 0.12) (type solid)) (layer "F.SilkS"))
  (fp_line (start -1.62 1.37) (end -1.62 -1.37) (stroke (width 0.12) (type solid)) (layer "F.SilkS"))
  (fp_line (start -1.62 -1.37) (end 6.62 -1.37) (stroke (width 0.12) (type solid)) (layer "F.SilkS"))
  (pad "1" thru_hole circle (at 0 0 180) (size 2 2) (drill 0.8) (layers "*.Cu" "*.Mask") (remove_unused_layers no) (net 11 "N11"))
  (pad "2" thru_hole circle (at 5 0 180) (size 2 2) (drill 0.8) (layers "*.Cu" "*.Mask") (remove_unused_layers no) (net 2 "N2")))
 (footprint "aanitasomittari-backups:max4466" (layer "B.Cu") (at 229.55 76.25 -90)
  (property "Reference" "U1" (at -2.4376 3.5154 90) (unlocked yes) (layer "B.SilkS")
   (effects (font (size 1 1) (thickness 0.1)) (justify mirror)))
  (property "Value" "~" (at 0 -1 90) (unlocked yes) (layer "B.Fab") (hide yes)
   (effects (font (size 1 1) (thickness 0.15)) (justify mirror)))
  (pad "1" thru_hole circle (at 5.2 1.3 180) (size 1.9304 1.9304) (drill 1) (layers "*.Cu" "*.Mask") (remove_unused_layers no)
   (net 10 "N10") (solder_mask_margin 0.0762) (thermal_bridge_angle 0))
  (pad "2" thru_hole circle (at 2.7 1.3 180) (size 1.9304 1.9304) (drill 1) (layers "*.Cu" "*.Mask") (remove_unused_layers no) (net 2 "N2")
   (solder_mask_margin 0.0762) (thermal_bridge_angle 0))
  (pad "3" thru_hole circle (at 0.2 1.3 180) (size 1.9304 1.9304) (drill 1) (layers "*.Cu" "*.Mask") (remove_unused_layers no)
   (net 21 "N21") (solder_mask_margin 0.0762) (thermal_bridge_angle 0)))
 (gr_rect (start 151.6 42.2) (end 240.3 97.35) (stroke (width 0.2) (type solid)) (fill no) (layer "Edge.Cuts"))
 (segment (start 164.3825 73.3) (end 164.3825 77.3675) (width 1) (layer "F.Cu") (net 2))
 (segment (start 214.1288 78.95) (end 228.25 78.95) (width 1) (layer "F.Cu") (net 2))
 (segment (start 162.0056 73.3) (end 164.3825 73.3) (width 1) (layer "F.Cu") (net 2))
 (segment (start 191.765 64.93) (end 200.1088 64.93) (width 1) (layer "F.Cu") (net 2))
 (segment (start 228.05 65.42) (end 230.12 65.42) (width 1) (layer "F.Cu") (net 2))
 (segment (start 160.15 90.4) (end 158.9 89.15) (width 1) (layer "F.Cu") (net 2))
 (segment (start 158.9 89.15) (end 158.9 76.4056) (width 1) (layer "F.Cu") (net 2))
 (segment (start 232.15 81.75) (end 223.5 90.4) (width 1) (layer "F.Cu") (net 2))
 (segment (start 232.1 78.95) (end 232.15 79) (width 1) (layer "F.Cu") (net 2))
 (segment (start 230.12 65.42) (end 232.15 67.45) (width 1) (layer "F.Cu") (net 2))
 (segment (start 162.05 86.8) (end 161.9 86.95) (width 1) (layer "F.Cu") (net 2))
 (segment (start 164.3825 68) (end 180.0818 68) (width 1) (layer "F.Cu") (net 2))
 (segment (start 228.05 57.95) (end 228.05 65.42) (width 1) (layer "F.Cu") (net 2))
 (segment (start 180.6118 67.47) (end 184.145 67.47) (width 1) (layer "F.Cu") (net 2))
 (segment (start 164.3825 68) (end 164.3825 73.3) (width 1) (layer "F.Cu") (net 2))
 (segment (start 200.1088 64.93) (end 214.1288 78.95) (width 1) (layer "F.Cu") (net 2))
 (segment (start 232.15 67.45) (end 232.15 79) (width 1) (layer "F.Cu") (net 2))
 (segment (start 223.5 90.4) (end 160.15 90.4) (width 1) (layer "F.Cu") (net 2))
 (segment (start 180.0818 68) (end 180.6118 67.47) (width 1) (layer "F.Cu") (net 2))
 (segment (start 164.3825 77.3675) (end 162.05 79.7) (width 1) (layer "F.Cu") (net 2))
 (segment (start 232.15 79) (end 232.15 81.75) (width 1) (layer "F.Cu") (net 2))
 (segment (start 228.05 50.48) (end 228.05 57.95) (width 1) (layer "F.Cu") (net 2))
 (segment (start 228.25 78.95) (end 232.1 78.95) (width 1) (layer "F.Cu") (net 2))
 (segment (start 162.05 79.7) (end 162.05 86.8) (width 1) (layer "F.Cu") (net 2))
 (segment (start 183.865 67.75) (end 184.145 67.47) (width 0.2) (layer "F.Cu") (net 2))
 (segment (start 158.9 76.4056) (end 162.0056 73.3) (width 1) (layer "F.Cu") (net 2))
 (segment (start 164.3825 63) (end 177.25 63) (width 1) (layer "F.Cu") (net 10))
 (segment (start 189.26 70.01) (end 188.1 68.85) (width 1) (layer "F.Cu") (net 10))
 (segment (start 177.25 63) (end 179.18 64.93) (width 1) (layer "F.Cu") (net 10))
 (segment (start 183.965 64.75) (end 184.145 64.93) (width 0.2) (layer "F.Cu") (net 10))
 (segment (start 186.03 64.93) (end 188.1 67) (width 1) (layer "F.Cu") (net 10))
 (segment (start 188.1 68.85) (end 188.1 67) (width 1) (layer "F.Cu") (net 10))
 (segment (start 191.765 70.01) (end 189.26 70.01) (width 1) (layer "F.Cu") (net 10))
 (segment (start 198.5848 70.01) (end 210.0248 81.45) (width 1) (layer "F.Cu") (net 10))
 (segment (start 191.765 70.01) (end 198.5848 70.01) (width 1) (layer "F.Cu") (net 10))
 (segment (start 188.1 67) (end 188.57 67.47) (width 1) (layer "F.Cu") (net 10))
 (segment (start 179.18 64.93) (end 184.145 64.93) (width 1) (layer "F.Cu") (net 10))
 (segment (start 184.145 64.93) (end 186.03 64.93) (width 1) (layer "F.Cu") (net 10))
 (segment (start 188.57 67.47) (end 191.765 67.47) (width 1) (layer "F.Cu") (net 10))
 (segment (start 210.0248 81.45) (end 228.25 81.45) (width 1) (layer "F.Cu") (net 10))
 (segment (start 191.765 62.39) (end 202.2932 62.39) (width 1) (layer "F.Cu") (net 21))
 (segment (start 202.2932 62.39) (end 216.3532 76.45) (width 1) (layer "F.Cu") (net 21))
 (segment (start 216.3532 76.45) (end 228.25 76.45) (width 1) (layer "F.Cu") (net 21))
 (segment (start 177.75 82.59) (end 177.75 75.95) (width 1) (layer "F.Cu") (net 11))
 (segment (start 177.75 75.95) (end 181.15 72.55) (width 1) (layer "F.Cu") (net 11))
 (segment (start 181.15 72.55) (end 184.145 72.55) (width 1) (layer "F.Cu") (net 11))
 (segment (start 175.1 85.24) (end 177.75 82.59) (width 1) (layer "F.Cu") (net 11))
 (segment (start 173.39 86.95) (end 175.1 85.24) (width 1) (layer "F.Cu") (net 11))
 (segment (start 166.9 86.95) (end 173.39 86.95) (width 1) (layer "F.Cu") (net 11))
 (segment (start 174.7388 80.7212) (end 175.1 80.36) (width 1) (layer "F.Cu") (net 1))
 (segment (start 168.0712 80.7212) (end 174.7388 80.7212) (width 1) (layer "F.Cu") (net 1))
 (segment (start 175.1 80.36) (end 175.1 73.947) (width 1) (layer "F.Cu") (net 1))
 (segment (start 179.037 70.01) (end 184.145 70.01) (width 1) (layer "F.Cu") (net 1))
 (segment (start 175.1 73.947) (end 179.037 70.01) (width 1) (layer "F.Cu") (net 1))
 (segment (start 167.05 79.7) (end 168.0712 80.7212) (width 1) (layer "F.Cu") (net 1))
 (segment (start 222 65.55) (end 225.38 65.55) (width 1) (layer "F.Cu") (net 3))
 (segment (start 225.38 65.55) (end 225.51 65.42) (width 1) (layer "F.Cu") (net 3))
 (segment (start 215.48 59.25) (end 218.15 59.25) (width 1) (layer "F.Cu") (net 3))
 (segment (start 219.95 63.5) (end 222 65.55) (width 1) (layer "F.Cu") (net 3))
 (segment (start 219.95 61.05) (end 219.95 63.5) (width 1) (layer "F.Cu") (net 3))
 (segment (start 218.15 59.25) (end 219.95 61.05) (width 1) (layer "F.Cu") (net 3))
 (segment (start 218.6 56.05) (end 220.55 58) (width 1) (layer "F.Cu") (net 28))
 (segment (start 215.53 56.05) (end 218.6 56.05) (width 1) (layer "F.Cu") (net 28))
 (segment (start 220.55 58) (end 225.46 58) (width 1) (layer "F.Cu") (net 28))
 (segment (start 225.46 58) (end 225.51 57.95) (width 1) (layer "F.Cu") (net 28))
 (segment (start 225.44 50.55) (end 225.51 50.48) (width 1) (layer "F.Cu") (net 27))
 (segment (start 221.95 50.55) (end 225.44 50.55) (width 1) (layer "F.Cu") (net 27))
 (segment (start 215.5 52.8) (end 219.7 52.8) (width 1) (layer "F.Cu") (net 27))
 (segment (start 219.7 52.8) (end 221.95 50.55) (width 1) (layer "F.Cu") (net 27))
 (segment (start 198.95 59.85) (end 199.55 59.25) (width 1) (layer "F.Cu") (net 22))
 (segment (start 191.765 59.85) (end 198.95 59.85) (width 1) (layer "F.Cu") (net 22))
 (segment (start 199.55 59.25) (end 205.32 59.25) (width 1) (layer "F.Cu") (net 22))
 (segment (start 191.765 57.31) (end 197.49 57.31) (width 1) (layer "F.Cu") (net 23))
 (segment (start 198.75 56.05) (end 205.37 56.05) (width 1) (layer "F.Cu") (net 23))
 (segment (start 197.49 57.31) (end 198.75 56.05) (width 1) (layer "F.Cu") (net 23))
 (segment (start 198.75 52.8) (end 205.34 52.8) (width 1) (layer "F.Cu") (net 24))
 (segment (start 191.765 54.77) (end 196.78 54.77) (width 1) (layer "F.Cu") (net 24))
 (segment (start 196.78 54.77) (end 198.75 52.8) (width 1) (layer "F.Cu") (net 24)))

